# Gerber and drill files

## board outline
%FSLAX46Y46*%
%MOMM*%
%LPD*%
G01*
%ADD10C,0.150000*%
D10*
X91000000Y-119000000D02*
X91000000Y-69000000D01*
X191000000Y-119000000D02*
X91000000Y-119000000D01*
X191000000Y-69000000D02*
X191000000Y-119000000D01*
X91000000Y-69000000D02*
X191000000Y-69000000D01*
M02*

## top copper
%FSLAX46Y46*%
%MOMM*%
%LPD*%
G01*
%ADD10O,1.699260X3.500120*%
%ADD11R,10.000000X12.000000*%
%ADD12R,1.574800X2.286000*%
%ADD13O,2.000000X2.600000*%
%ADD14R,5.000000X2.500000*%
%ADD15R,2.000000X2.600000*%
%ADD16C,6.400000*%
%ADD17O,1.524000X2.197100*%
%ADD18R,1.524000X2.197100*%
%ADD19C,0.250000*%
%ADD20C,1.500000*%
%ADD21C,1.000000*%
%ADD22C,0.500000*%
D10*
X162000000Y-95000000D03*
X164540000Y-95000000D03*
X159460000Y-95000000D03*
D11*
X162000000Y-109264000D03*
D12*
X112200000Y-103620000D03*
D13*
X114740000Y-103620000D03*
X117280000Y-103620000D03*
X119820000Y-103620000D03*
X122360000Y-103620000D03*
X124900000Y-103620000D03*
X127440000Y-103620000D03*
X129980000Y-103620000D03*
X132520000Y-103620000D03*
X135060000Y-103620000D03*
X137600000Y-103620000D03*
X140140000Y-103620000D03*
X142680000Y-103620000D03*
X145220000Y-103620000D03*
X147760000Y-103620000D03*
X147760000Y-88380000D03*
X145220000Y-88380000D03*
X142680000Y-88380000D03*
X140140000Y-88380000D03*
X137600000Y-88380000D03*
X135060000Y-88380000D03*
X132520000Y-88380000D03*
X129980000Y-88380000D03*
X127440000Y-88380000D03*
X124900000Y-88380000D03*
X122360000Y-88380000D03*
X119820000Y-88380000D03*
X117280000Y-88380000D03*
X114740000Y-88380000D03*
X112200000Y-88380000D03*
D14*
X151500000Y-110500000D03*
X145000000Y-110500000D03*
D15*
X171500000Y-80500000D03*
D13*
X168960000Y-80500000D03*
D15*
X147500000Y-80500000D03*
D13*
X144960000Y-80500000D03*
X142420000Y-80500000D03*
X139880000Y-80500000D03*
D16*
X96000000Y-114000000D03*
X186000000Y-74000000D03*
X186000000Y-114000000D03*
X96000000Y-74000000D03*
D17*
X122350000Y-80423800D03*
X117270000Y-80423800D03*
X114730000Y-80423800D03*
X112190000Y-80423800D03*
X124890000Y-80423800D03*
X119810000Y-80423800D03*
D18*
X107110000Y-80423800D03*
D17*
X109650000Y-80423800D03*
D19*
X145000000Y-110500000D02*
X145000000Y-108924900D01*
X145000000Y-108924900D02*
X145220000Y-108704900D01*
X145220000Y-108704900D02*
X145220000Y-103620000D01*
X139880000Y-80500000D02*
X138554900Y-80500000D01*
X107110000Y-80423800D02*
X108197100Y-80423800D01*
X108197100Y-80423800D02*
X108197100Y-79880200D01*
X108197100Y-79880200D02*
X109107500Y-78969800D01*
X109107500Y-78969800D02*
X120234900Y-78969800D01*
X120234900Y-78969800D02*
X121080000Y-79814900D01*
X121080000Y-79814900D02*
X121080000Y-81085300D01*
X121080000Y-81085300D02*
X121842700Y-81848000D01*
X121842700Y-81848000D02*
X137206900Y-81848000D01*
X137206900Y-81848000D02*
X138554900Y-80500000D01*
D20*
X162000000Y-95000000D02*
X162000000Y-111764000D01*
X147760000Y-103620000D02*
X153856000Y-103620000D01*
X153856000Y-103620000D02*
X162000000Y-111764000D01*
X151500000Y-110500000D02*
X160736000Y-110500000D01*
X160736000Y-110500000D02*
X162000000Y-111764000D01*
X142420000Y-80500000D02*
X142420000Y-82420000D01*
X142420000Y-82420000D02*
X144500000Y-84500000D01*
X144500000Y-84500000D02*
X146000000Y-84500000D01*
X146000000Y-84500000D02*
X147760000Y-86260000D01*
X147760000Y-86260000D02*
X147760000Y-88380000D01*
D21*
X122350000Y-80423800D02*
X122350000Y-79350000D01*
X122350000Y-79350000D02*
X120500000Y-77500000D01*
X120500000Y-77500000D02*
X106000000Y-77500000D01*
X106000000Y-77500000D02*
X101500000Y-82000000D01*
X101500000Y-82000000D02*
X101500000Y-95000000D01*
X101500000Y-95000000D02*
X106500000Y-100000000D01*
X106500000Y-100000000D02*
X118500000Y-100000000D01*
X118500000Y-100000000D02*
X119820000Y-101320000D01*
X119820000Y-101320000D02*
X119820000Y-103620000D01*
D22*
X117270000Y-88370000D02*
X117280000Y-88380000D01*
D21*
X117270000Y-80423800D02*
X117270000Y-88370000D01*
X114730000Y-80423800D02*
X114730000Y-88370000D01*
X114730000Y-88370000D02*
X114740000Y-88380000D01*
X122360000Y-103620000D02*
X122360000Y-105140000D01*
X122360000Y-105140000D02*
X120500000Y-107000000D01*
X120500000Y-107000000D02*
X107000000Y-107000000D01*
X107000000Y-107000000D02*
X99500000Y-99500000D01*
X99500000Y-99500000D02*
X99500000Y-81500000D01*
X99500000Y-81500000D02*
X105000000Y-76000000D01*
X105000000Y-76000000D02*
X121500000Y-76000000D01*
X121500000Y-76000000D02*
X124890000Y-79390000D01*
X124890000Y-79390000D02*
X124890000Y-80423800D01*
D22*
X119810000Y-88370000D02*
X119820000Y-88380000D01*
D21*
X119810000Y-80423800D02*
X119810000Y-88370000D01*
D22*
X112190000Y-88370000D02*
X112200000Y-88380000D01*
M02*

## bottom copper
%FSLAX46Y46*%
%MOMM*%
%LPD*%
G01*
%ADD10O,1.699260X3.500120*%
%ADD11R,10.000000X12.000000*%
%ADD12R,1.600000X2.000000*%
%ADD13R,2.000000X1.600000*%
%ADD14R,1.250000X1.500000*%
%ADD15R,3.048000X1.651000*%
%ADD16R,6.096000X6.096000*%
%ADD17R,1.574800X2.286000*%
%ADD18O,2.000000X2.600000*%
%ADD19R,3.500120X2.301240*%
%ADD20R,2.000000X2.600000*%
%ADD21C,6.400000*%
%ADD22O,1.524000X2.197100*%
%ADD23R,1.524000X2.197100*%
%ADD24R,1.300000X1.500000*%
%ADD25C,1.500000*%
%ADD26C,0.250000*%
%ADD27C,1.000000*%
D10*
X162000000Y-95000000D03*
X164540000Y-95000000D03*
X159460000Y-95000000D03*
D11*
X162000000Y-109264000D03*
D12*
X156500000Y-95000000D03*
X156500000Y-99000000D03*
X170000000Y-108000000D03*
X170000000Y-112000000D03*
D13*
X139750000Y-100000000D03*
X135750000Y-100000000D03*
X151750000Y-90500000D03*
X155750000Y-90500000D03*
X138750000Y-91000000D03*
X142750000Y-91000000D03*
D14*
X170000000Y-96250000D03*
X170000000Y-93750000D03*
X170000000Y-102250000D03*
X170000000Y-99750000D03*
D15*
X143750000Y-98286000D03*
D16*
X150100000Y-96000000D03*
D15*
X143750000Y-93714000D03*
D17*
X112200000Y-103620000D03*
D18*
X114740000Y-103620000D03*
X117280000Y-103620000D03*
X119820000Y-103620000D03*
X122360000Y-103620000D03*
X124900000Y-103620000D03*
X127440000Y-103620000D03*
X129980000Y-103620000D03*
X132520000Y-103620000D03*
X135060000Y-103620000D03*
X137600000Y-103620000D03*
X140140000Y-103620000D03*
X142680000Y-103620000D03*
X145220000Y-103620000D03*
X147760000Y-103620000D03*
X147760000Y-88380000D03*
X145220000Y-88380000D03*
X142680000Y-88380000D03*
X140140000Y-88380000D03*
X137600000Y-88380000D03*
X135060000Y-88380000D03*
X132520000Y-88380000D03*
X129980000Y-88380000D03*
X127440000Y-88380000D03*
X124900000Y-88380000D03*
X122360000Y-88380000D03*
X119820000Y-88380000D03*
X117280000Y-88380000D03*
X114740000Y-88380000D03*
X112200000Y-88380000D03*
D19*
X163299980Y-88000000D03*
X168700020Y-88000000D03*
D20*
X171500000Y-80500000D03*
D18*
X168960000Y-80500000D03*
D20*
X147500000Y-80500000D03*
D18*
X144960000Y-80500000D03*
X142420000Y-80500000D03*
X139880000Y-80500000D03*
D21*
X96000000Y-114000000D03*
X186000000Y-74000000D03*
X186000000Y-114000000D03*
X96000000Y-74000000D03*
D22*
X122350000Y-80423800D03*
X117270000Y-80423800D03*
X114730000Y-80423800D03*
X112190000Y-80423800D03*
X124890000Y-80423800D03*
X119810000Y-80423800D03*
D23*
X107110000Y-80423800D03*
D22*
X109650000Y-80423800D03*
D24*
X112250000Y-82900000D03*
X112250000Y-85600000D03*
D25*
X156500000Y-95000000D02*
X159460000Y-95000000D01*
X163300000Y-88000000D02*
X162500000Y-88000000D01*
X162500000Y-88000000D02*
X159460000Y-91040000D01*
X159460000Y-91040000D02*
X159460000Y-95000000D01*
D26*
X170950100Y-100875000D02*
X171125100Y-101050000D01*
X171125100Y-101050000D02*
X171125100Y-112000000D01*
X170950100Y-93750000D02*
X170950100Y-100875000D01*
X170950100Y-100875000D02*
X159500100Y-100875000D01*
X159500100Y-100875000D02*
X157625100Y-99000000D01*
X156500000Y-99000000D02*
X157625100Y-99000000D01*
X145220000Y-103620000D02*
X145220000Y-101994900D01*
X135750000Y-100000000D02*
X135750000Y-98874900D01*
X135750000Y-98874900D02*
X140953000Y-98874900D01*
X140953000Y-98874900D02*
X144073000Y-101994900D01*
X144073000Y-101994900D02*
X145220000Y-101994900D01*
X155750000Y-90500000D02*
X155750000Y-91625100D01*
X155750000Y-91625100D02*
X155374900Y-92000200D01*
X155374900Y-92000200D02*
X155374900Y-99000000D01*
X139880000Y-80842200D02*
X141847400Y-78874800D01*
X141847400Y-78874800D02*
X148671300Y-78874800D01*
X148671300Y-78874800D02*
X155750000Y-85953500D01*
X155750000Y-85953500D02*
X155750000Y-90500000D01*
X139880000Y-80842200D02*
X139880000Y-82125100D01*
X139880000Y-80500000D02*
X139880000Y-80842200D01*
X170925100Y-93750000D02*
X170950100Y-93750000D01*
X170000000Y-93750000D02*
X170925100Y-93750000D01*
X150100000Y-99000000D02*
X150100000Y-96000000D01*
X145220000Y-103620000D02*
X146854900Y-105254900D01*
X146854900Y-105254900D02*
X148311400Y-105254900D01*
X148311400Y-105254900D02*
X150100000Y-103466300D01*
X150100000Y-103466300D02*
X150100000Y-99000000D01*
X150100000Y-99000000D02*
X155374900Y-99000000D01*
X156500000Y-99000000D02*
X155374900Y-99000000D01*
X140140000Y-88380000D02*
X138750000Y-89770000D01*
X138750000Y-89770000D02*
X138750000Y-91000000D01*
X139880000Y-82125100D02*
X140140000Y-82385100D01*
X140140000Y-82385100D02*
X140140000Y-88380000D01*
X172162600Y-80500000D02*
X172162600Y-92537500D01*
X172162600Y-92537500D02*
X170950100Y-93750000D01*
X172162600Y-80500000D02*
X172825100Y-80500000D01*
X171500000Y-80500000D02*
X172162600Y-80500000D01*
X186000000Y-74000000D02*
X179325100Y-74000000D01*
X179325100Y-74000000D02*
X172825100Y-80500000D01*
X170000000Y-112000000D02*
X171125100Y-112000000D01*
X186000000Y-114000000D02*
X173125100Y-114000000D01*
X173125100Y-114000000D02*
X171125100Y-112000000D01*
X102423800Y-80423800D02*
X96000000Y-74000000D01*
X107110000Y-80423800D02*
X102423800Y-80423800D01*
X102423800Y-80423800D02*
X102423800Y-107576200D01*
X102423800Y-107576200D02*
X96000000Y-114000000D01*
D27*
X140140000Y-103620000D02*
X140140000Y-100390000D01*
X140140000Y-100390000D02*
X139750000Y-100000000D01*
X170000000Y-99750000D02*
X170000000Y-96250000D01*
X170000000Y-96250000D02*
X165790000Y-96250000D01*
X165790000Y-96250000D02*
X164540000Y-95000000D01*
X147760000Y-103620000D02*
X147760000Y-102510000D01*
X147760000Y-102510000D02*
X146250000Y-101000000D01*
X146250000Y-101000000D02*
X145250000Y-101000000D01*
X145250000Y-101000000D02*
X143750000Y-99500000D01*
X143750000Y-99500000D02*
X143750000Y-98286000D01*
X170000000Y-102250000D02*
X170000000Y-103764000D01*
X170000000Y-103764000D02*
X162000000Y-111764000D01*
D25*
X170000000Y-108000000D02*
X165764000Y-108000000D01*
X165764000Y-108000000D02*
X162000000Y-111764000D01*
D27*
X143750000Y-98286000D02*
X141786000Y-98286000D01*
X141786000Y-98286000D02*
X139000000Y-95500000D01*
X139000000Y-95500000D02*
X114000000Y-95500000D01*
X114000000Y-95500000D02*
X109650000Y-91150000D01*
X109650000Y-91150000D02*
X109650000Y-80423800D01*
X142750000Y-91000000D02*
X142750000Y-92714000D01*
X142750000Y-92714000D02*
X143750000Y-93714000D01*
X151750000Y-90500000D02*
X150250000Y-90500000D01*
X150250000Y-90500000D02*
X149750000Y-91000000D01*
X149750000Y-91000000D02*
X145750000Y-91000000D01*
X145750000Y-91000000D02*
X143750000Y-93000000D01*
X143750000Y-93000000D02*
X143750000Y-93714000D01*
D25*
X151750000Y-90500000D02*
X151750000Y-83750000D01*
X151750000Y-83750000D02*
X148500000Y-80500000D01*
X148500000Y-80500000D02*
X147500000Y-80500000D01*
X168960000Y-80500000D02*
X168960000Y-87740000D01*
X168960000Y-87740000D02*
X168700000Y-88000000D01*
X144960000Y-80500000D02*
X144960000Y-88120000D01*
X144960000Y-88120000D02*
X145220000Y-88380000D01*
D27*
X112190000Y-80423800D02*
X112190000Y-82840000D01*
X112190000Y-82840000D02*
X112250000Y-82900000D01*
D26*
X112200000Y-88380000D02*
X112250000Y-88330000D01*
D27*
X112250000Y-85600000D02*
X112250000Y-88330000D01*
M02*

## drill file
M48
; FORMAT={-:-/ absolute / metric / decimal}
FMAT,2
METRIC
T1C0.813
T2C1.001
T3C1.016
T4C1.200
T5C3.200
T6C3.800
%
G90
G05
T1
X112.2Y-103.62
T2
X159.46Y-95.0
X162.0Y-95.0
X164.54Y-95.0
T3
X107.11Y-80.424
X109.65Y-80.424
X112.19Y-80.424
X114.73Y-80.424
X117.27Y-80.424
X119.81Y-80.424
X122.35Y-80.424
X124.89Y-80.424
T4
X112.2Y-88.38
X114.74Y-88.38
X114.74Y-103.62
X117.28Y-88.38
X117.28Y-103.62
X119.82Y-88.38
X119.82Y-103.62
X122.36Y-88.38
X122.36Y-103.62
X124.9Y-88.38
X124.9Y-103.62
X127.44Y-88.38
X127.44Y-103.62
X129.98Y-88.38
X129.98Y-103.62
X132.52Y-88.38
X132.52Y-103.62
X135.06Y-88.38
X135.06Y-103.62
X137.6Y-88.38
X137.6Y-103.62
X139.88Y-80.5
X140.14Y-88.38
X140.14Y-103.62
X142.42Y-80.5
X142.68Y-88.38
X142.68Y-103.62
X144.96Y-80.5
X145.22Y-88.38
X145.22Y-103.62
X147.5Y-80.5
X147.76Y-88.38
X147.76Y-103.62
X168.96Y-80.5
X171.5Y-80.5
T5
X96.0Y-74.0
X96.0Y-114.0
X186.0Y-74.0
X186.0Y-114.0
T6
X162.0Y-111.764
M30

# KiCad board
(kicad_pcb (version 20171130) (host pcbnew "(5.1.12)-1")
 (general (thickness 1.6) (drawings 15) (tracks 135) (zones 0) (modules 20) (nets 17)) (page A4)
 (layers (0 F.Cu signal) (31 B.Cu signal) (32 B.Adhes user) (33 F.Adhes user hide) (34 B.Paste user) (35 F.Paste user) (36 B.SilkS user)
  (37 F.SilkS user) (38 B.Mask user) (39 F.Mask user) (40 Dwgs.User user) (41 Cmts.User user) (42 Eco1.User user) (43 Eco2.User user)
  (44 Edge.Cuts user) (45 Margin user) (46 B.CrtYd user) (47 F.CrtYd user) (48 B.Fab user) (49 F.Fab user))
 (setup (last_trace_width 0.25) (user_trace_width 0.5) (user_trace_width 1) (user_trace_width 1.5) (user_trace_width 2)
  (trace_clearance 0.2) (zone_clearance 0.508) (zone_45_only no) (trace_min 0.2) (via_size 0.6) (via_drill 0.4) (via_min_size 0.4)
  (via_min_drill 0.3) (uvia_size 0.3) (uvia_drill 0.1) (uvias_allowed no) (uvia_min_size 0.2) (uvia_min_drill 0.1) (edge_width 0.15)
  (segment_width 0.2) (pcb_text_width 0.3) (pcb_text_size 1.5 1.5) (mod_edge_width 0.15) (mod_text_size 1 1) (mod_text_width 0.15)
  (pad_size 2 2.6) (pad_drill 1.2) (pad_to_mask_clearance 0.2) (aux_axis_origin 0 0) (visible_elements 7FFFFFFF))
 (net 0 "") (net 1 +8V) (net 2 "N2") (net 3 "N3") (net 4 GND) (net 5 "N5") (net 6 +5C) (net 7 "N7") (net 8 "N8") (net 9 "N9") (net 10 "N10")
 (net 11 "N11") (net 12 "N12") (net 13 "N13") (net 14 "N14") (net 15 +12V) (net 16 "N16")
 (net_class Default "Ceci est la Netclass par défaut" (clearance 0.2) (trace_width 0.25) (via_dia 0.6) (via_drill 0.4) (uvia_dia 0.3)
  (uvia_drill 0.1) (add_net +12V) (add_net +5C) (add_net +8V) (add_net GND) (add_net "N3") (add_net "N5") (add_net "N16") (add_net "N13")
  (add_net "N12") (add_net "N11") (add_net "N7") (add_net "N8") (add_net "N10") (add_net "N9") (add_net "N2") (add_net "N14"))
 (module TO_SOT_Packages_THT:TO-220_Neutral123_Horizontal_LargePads (layer F.Cu) (at 162 95 180)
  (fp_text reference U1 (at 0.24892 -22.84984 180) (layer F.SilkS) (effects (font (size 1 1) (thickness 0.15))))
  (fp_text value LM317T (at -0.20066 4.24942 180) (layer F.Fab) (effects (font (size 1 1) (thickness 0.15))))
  (pad 2 thru_hole oval (at 0 0 270) (size 3.50012 1.69926) (drill 1.00076) (layers *.Cu *.Mask F.SilkS) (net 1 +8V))
  (pad 1 thru_hole oval (at -2.54 0 270) (size 3.50012 1.69926) (drill 1.00076) (layers *.Cu *.Mask F.SilkS) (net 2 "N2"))
  (pad 3 thru_hole oval (at 2.54 0 270) (size 3.50012 1.69926) (drill 1.00076) (layers *.Cu *.Mask F.SilkS) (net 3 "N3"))
  (pad 2 thru_hole rect (at 0 -16.764 270) (size 12 10) (drill 3.79984 (offset -2.5 0)) (layers *.Cu *.Paste *.Mask) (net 1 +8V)))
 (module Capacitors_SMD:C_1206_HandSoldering (layer B.Cu) (at 156.5 97 270)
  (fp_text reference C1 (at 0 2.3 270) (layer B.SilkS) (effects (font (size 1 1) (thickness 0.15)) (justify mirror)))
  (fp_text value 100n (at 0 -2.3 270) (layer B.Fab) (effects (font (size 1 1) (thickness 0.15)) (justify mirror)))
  (pad 1 smd rect (at -2 0 270) (size 2 1.6) (layers B.Cu B.Paste B.Mask) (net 3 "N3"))
  (pad 2 smd rect (at 2 0 270) (size 2 1.6) (layers B.Cu B.Paste B.Mask) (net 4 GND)))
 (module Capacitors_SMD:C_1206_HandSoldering (layer B.Cu) (at 170 110 270)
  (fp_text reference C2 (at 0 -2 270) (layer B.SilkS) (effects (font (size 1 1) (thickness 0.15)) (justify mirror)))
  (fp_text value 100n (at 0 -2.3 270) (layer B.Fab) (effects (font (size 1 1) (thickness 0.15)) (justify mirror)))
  (pad 1 smd rect (at -2 0 270) (size 2 1.6) (layers B.Cu B.Paste B.Mask) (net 1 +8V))
  (pad 2 smd rect (at 2 0 270) (size 2 1.6) (layers B.Cu B.Paste B.Mask) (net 4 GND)))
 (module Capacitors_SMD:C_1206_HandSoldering (layer B.Cu) (at 137.75 100 180)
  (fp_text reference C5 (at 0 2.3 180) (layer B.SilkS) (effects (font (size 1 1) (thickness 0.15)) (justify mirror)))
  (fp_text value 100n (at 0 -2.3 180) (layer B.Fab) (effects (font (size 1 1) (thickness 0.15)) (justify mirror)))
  (pad 1 smd rect (at -2 0 180) (size 2 1.6) (layers B.Cu B.Paste B.Mask) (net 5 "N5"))
  (pad 2 smd rect (at 2 0 180) (size 2 1.6) (layers B.Cu B.Paste B.Mask) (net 4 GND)))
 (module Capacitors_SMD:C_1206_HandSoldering (layer B.Cu) (at 153.75 90.5)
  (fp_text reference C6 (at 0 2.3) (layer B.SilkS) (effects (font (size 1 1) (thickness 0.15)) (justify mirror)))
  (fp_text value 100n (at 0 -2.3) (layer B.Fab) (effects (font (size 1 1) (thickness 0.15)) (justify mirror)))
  (pad 1 smd rect (at -2 0) (size 2 1.6) (layers B.Cu B.Paste B.Mask) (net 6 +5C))
  (pad 2 smd rect (at 2 0) (size 2 1.6) (layers B.Cu B.Paste B.Mask) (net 4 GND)))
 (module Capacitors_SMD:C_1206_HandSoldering (layer B.Cu) (at 140.75 91)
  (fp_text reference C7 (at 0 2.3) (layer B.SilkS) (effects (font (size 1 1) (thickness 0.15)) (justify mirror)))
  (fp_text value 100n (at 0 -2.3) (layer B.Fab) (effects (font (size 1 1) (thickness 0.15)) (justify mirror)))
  (pad 1 smd rect (at -2 0) (size 2 1.6) (layers B.Cu B.Paste B.Mask) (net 4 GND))
  (pad 2 smd rect (at 2 0) (size 2 1.6) (layers B.Cu B.Paste B.Mask) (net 6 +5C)))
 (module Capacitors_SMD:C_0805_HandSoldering (layer B.Cu) (at 170 95 90)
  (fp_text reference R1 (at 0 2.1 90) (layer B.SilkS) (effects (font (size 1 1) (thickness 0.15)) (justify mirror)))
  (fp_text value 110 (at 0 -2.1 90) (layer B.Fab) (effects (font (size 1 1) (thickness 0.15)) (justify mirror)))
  (pad 1 smd rect (at -1.25 0 90) (size 1.5 1.25) (layers B.Cu B.Paste B.Mask) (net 2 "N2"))
  (pad 2 smd rect (at 1.25 0 90) (size 1.5 1.25) (layers B.Cu B.Paste B.Mask) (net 4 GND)))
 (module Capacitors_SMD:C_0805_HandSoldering (layer B.Cu) (at 170 101 90)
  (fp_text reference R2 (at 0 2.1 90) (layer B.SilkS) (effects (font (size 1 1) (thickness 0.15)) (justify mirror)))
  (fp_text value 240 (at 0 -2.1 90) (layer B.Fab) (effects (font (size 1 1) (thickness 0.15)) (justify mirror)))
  (pad 1 smd rect (at -1.25 0 90) (size 1.5 1.25) (layers B.Cu B.Paste B.Mask) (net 1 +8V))
  (pad 2 smd rect (at 1.25 0 90) (size 1.5 1.25) (layers B.Cu B.Paste B.Mask) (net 2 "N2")))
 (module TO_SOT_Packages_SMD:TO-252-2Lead (layer B.Cu) (at 143.75 96 90)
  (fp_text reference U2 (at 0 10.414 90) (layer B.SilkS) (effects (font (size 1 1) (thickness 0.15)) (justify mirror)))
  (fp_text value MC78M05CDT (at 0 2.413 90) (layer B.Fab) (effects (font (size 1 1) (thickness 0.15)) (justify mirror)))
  (pad 1 smd rect (at -2.286 0 90) (size 1.651 3.048) (layers B.Cu B.Paste B.Mask) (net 1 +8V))
  (pad 2 smd rect (at 0 6.35 90) (size 6.096 6.096) (layers B.Cu B.Paste B.Mask) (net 4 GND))
  (pad 3 smd rect (at 2.286 0 90) (size 1.651 3.048) (layers B.Cu B.Paste B.Mask) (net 6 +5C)))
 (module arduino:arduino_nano (layer F.Cu) (at 131.25 96)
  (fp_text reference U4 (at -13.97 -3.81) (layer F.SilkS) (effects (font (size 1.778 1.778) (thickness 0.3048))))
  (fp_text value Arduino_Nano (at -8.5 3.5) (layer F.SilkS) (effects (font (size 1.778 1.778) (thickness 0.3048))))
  (pad 1 thru_hole rect (at -19.05 7.62) (size 1.5748 2.286) (drill 0.8128) (layers *.Cu *.Mask F.SilkS))
  (pad 2 thru_hole oval (at -16.51 7.62) (size 2 2.6) (drill 1.2) (layers *.Cu *.Mask F.SilkS))
  (pad 3 thru_hole oval (at -13.97 7.62) (size 2 2.6) (drill 1.2) (layers *.Cu *.Mask F.SilkS))
  (pad 4 thru_hole oval (at -11.43 7.62) (size 2 2.6) (drill 1.2) (layers *.Cu *.Mask F.SilkS) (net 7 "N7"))
  (pad 5 thru_hole oval (at -8.89 7.62) (size 2 2.6) (drill 1.2) (layers *.Cu *.Mask F.SilkS) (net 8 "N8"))
  (pad 6 thru_hole oval (at -6.35 7.62) (size 2 2.6) (drill 1.2) (layers *.Cu *.Mask F.SilkS))
  (pad 7 thru_hole oval (at -3.81 7.62) (size 2 2.6) (drill 1.2) (layers *.Cu *.Mask F.SilkS))
  (pad 8 thru_hole oval (at -1.27 7.62) (size 2 2.6) (drill 1.2) (layers *.Cu *.Mask F.SilkS))
  (pad 9 thru_hole oval (at 1.27 7.62) (size 2 2.6) (drill 1.2) (layers *.Cu *.Mask F.SilkS))
  (pad 10 thru_hole oval (at 3.81 7.62) (size 2 2.6) (drill 1.2) (layers *.Cu *.Mask F.SilkS))
  (pad 11 thru_hole oval (at 6.35 7.62) (size 2 2.6) (drill 1.2) (layers *.Cu *.Mask F.SilkS))
  (pad 12 thru_hole oval (at 8.89 7.62) (size 2 2.6) (drill 1.2) (layers *.Cu *.Mask F.SilkS) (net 5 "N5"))
  (pad 13 thru_hole oval (at 11.43 7.62) (size 2 2.6) (drill 1.2) (layers *.Cu *.Mask F.SilkS))
  (pad 14 thru_hole oval (at 13.97 7.62) (size 2 2.6) (drill 1.2) (layers *.Cu *.Mask F.SilkS) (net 4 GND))
  (pad 15 thru_hole oval (at 16.51 7.62) (size 2 2.6) (drill 1.2) (layers *.Cu *.Mask F.SilkS) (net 1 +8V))
  (pad 16 thru_hole oval (at 16.51 -7.62) (size 2 2.6) (drill 1.2) (layers *.Cu *.Mask F.SilkS) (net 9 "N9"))
  (pad 17 thru_hole oval (at 13.97 -7.62) (size 2 2.6) (drill 1.2) (layers *.Cu *.Mask F.SilkS) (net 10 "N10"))
  (pad 18 thru_hole oval (at 11.43 -7.62) (size 2 2.6) (drill 1.2) (layers *.Cu *.Mask F.SilkS))
  (pad 19 thru_hole oval (at 8.89 -7.62) (size 2 2.6) (drill 1.2) (layers *.Cu *.Mask F.SilkS) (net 4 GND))
  (pad 20 thru_hole oval (at 6.35 -7.62) (size 2 2.6) (drill 1.2) (layers *.Cu *.Mask F.SilkS))
  (pad 21 thru_hole oval (at 3.81 -7.62) (size 2 2.6) (drill 1.2) (layers *.Cu *.Mask F.SilkS))
  (pad 22 thru_hole oval (at 1.27 -7.62) (size 2 2.6) (drill 1.2) (layers *.Cu *.Mask F.SilkS))
  (pad 23 thru_hole oval (at -1.27 -7.62) (size 2 2.6) (drill 1.2) (layers *.Cu *.Mask F.SilkS))
  (pad 24 thru_hole oval (at -3.81 -7.62) (size 2 2.6) (drill 1.2) (layers *.Cu *.Mask F.SilkS))
  (pad 25 thru_hole oval (at -6.35 -7.62) (size 2 2.6) (drill 1.2) (layers *.Cu *.Mask F.SilkS))
  (pad 26 thru_hole oval (at -8.89 -7.62) (size 2 2.6) (drill 1.2) (layers *.Cu *.Mask F.SilkS))
  (pad 27 thru_hole oval (at -11.43 -7.62) (size 2 2.6) (drill 1.2) (layers *.Cu *.Mask F.SilkS) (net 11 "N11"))
  (pad 28 thru_hole oval (at -13.97 -7.62) (size 2 2.6) (drill 1.2) (layers *.Cu *.Mask F.SilkS) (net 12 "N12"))
  (pad 29 thru_hole oval (at -16.51 -7.62) (size 2 2.6) (drill 1.2) (layers *.Cu *.Mask F.SilkS) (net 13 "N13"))
  (pad 30 thru_hole oval (at -19.05 -7.62) (size 2 2.6) (drill 1.2) (layers *.Cu *.Mask F.SilkS) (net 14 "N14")))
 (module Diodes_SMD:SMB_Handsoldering (layer B.Cu) (at 166 88)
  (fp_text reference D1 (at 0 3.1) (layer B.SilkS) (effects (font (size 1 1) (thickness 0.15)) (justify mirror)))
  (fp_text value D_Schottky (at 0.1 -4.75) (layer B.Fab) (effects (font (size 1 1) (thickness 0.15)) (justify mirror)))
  (pad 1 smd rect (at -2.70002 0) (size 3.50012 2.30124) (layers B.Cu B.Paste B.Mask) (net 3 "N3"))
  (pad 2 smd rect (at 2.70002 0) (size 3.50012 2.30124) (layers B.Cu B.Paste B.Mask) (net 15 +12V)))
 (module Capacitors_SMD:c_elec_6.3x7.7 (layer F.Cu) (at 148.5 110.5)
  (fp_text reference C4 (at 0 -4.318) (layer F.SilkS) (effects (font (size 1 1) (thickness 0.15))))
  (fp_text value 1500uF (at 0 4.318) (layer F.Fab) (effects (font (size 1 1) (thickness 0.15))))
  (pad 1 smd rect (at 3 0) (size 5 2.5) (layers F.Cu F.Paste F.Mask) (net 1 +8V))
  (pad 2 smd rect (at -3.5 0) (size 5 2.5) (layers F.Cu F.Paste F.Mask) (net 4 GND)))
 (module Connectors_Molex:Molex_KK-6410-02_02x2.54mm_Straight (layer F.Cu) (at 171.5 80.5 180)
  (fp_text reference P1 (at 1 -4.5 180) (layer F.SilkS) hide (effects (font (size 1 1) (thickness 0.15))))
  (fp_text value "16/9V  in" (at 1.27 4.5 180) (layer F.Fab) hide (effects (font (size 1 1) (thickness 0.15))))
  (pad 1 thru_hole rect (at 0 0 180) (size 2 2.6) (drill 1.2) (layers *.Cu *.Mask) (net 4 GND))
  (pad 2 thru_hole oval (at 2.54 0 180) (size 2 2.6) (drill 1.2) (layers *.Cu *.Mask) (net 15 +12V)))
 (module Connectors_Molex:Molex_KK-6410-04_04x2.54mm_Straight (layer F.Cu) (at 147.5 80.5 180)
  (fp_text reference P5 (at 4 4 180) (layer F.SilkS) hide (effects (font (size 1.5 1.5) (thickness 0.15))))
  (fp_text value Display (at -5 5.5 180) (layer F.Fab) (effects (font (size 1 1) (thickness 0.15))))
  (pad 1 thru_hole rect (at 0 0 180) (size 2 2.6) (drill 1.2) (layers *.Cu *.Mask) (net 6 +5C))
  (pad 2 thru_hole oval (at 2.54 0 180) (size 2 2.6) (drill 1.2) (layers *.Cu *.Mask) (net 10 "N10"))
  (pad 3 thru_hole oval (at 5.08 0 180) (size 2 2.6) (drill 1.2) (layers *.Cu *.Mask) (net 9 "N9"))
  (pad 4 thru_hole oval (at 7.62 0 180) (size 2 2.6) (drill 1.2) (layers *.Cu *.Mask) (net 4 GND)))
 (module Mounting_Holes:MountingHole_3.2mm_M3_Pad (layer F.Cu) (at 96 114)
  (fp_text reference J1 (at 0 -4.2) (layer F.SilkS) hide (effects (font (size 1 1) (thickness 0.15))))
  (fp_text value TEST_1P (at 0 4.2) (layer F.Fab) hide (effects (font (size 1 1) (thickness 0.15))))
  (pad 1 thru_hole circle (at 0 0) (size 6.4 6.4) (drill 3.2) (layers *.Cu *.Mask) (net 4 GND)))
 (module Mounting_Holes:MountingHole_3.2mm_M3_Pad (layer F.Cu) (at 186 74)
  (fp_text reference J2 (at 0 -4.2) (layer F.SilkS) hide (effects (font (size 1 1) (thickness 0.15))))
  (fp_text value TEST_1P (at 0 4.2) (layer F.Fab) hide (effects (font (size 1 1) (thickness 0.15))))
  (pad 1 thru_hole circle (at 0 0) (size 6.4 6.4) (drill 3.2) (layers *.Cu *.Mask) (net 4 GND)))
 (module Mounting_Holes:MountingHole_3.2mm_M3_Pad (layer F.Cu) (at 186 114)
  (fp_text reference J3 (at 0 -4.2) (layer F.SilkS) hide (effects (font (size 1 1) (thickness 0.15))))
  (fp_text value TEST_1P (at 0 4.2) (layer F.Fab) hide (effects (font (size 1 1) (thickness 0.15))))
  (pad 1 thru_hole circle (at 0 0) (size 6.4 6.4) (drill 3.2) (layers *.Cu *.Mask) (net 4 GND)))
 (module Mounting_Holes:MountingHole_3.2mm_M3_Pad (layer F.Cu) (at 96 74)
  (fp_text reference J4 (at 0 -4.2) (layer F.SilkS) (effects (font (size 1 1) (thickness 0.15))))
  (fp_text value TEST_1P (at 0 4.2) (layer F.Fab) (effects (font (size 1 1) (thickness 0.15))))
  (pad 1 thru_hole circle (at 0 0) (size 6.4 6.4) (drill 3.2) (layers *.Cu *.Mask) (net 4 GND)))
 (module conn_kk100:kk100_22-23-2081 (layer F.Cu) (at 116 80.5)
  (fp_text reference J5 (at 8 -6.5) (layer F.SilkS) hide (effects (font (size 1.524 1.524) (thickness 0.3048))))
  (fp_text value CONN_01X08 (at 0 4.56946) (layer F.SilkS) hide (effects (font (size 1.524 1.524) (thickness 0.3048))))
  (pad 7 thru_hole oval (at 6.35 -0.0762) (size 1.524 2.1971) (drill 1.016) (layers *.Cu *.Mask F.SilkS) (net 7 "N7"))
  (pad 5 thru_hole oval (at 1.27 -0.0762) (size 1.524 2.1971) (drill 1.016) (layers *.Cu *.Mask F.SilkS) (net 12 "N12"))
  (pad 4 thru_hole oval (at -1.27 -0.0762) (size 1.524 2.1971) (drill 1.016) (layers *.Cu *.Mask F.SilkS) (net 13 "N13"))
  (pad 3 thru_hole oval (at -3.81 -0.0762) (size 1.524 2.1971) (drill 1.016) (layers *.Cu *.Mask F.SilkS) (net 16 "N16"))
  (pad 8 thru_hole oval (at 8.89 -0.0762) (size 1.524 2.1971) (drill 1.016) (layers *.Cu *.Mask F.SilkS) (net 8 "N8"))
  (pad 6 thru_hole oval (at 3.81 -0.0762) (size 1.524 2.1971) (drill 1.016) (layers *.Cu *.Mask F.SilkS) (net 11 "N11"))
  (pad 1 thru_hole rect (at -8.89 -0.0762) (size 1.524 2.1971) (drill 1.016) (layers *.Cu *.Mask F.SilkS) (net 4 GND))
  (pad 2 thru_hole oval (at -6.35 -0.0762) (size 1.524 2.1971) (drill 1.016) (layers *.Cu *.Mask F.SilkS) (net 1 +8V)))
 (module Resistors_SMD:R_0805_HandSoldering (layer B.Cu) (at 112.25 84.25 270)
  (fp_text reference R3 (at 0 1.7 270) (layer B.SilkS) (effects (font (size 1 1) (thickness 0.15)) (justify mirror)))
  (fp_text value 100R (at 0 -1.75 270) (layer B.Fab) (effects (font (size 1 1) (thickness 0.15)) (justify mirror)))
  (pad 1 smd rect (at -1.35 0 270) (size 1.5 1.3) (layers B.Cu B.Paste B.Mask) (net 16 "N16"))
  (pad 2 smd rect (at 1.35 0 270) (size 1.5 1.3) (layers B.Cu B.Paste B.Mask) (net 14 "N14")))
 (gr_line (start 91 119) (end 91 69) (angle 90) (layer Edge.Cuts) (width 0.15))
 (gr_line (start 191 119) (end 91 119) (angle 90) (layer Edge.Cuts) (width 0.15))
 (gr_line (start 191 69) (end 191 119) (angle 90) (layer Edge.Cuts) (width 0.15))
 (gr_line (start 91 69) (end 191 69) (angle 90) (layer Edge.Cuts) (width 0.15))
 (segment (start 156.5 95) (end 159.46 95) (width 1.5) (layer B.Cu) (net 3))
 (segment (start 163.3 88) (end 162.5 88) (width 1.5) (layer B.Cu) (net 3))
 (segment (start 162.5 88) (end 159.46 91.04) (width 1.5) (layer B.Cu) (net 3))
 (segment (start 159.46 91.04) (end 159.46 95) (width 1.5) (layer B.Cu) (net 3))
 (segment (start 170.9501 100.875) (end 171.1251 101.05) (width 0.25) (layer B.Cu) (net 4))
 (segment (start 171.1251 101.05) (end 171.1251 112) (width 0.25) (layer B.Cu) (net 4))
 (segment (start 170.9501 93.75) (end 170.9501 100.875) (width 0.25) (layer B.Cu) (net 4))
 (segment (start 170.9501 100.875) (end 159.5001 100.875) (width 0.25) (layer B.Cu) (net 4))
 (segment (start 159.5001 100.875) (end 157.6251 99) (width 0.25) (layer B.Cu) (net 4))
 (segment (start 156.5 99) (end 157.6251 99) (width 0.25) (layer B.Cu) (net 4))
 (segment (start 145.22 103.62) (end 145.22 101.9949) (width 0.25) (layer B.Cu) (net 4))
 (segment (start 135.75 100) (end 135.75 98.8749) (width 0.25) (layer B.Cu) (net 4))
 (segment (start 135.75 98.8749) (end 140.953 98.8749) (width 0.25) (layer B.Cu) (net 4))
 (segment (start 140.953 98.8749) (end 144.073 101.9949) (width 0.25) (layer B.Cu) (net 4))
 (segment (start 144.073 101.9949) (end 145.22 101.9949) (width 0.25) (layer B.Cu) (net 4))
 (segment (start 155.75 90.5) (end 155.75 91.6251) (width 0.25) (layer B.Cu) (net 4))
 (segment (start 155.75 91.6251) (end 155.3749 92.0002) (width 0.25) (layer B.Cu) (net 4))
 (segment (start 155.3749 92.0002) (end 155.3749 99) (width 0.25) (layer B.Cu) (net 4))
 (segment (start 139.88 80.8422) (end 141.8474 78.8748) (width 0.25) (layer B.Cu) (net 4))
 (segment (start 141.8474 78.8748) (end 148.6713 78.8748) (width 0.25) (layer B.Cu) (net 4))
 (segment (start 148.6713 78.8748) (end 155.75 85.9535) (width 0.25) (layer B.Cu) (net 4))
 (segment (start 155.75 85.9535) (end 155.75 90.5) (width 0.25) (layer B.Cu) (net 4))
 (segment (start 139.88 80.8422) (end 139.88 82.1251) (width 0.25) (layer B.Cu) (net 4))
 (segment (start 139.88 80.5) (end 139.88 80.8422) (width 0.25) (layer B.Cu) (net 4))
 (segment (start 170.9251 93.75) (end 170.9501 93.75) (width 0.25) (layer B.Cu) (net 4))
 (segment (start 170 93.75) (end 170.9251 93.75) (width 0.25) (layer B.Cu) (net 4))
 (segment (start 150.1 99) (end 150.1 96) (width 0.25) (layer B.Cu) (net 4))
 (segment (start 145.22 103.62) (end 146.8549 105.2549) (width 0.25) (layer B.Cu) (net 4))
 (segment (start 146.8549 105.2549) (end 148.3114 105.2549) (width 0.25) (layer B.Cu) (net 4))
 (segment (start 148.3114 105.2549) (end 150.1 103.4663) (width 0.25) (layer B.Cu) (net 4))
 (segment (start 150.1 103.4663) (end 150.1 99) (width 0.25) (layer B.Cu) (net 4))
 (segment (start 150.1 99) (end 155.3749 99) (width 0.25) (layer B.Cu) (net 4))
 (segment (start 156.5 99) (end 155.3749 99) (width 0.25) (layer B.Cu) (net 4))
 (segment (start 140.14 88.38) (end 138.75 89.77) (width 0.25) (layer B.Cu) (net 4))
 (segment (start 138.75 89.77) (end 138.75 91) (width 0.25) (layer B.Cu) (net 4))
 (segment (start 139.88 82.1251) (end 140.14 82.3851) (width 0.25) (layer B.Cu) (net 4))
 (segment (start 140.14 82.3851) (end 140.14 88.38) (width 0.25) (layer B.Cu) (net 4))
 (segment (start 145 110.5) (end 145 108.9249) (width 0.25) (layer F.Cu) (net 4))
 (segment (start 145 108.9249) (end 145.22 108.7049) (width 0.25) (layer F.Cu) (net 4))
 (segment (start 145.22 108.7049) (end 145.22 103.62) (width 0.25) (layer F.Cu) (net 4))
 (segment (start 172.1626 80.5) (end 172.1626 92.5375) (width 0.25) (layer B.Cu) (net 4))
 (segment (start 172.1626 92.5375) (end 170.9501 93.75) (width 0.25) (layer B.Cu) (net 4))
 (segment (start 172.1626 80.5) (end 172.8251 80.5) (width 0.25) (layer B.Cu) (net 4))
 (segment (start 171.5 80.5) (end 172.1626 80.5) (width 0.25) (layer B.Cu) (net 4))
 (segment (start 139.88 80.5) (end 138.5549 80.5) (width 0.25) (layer F.Cu) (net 4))
 (segment (start 107.11 80.4238) (end 108.1971 80.4238) (width 0.25) (layer F.Cu) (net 4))
 (segment (start 108.1971 80.4238) (end 108.1971 79.8802) (width 0.25) (layer F.Cu) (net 4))
 (segment (start 108.1971 79.8802) (end 109.1075 78.9698) (width 0.25) (layer F.Cu) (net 4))
 (segment (start 109.1075 78.9698) (end 120.2349 78.9698) (width 0.25) (layer F.Cu) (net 4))
 (segment (start 120.2349 78.9698) (end 121.08 79.8149) (width 0.25) (layer F.Cu) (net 4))
 (segment (start 121.08 79.8149) (end 121.08 81.0853) (width 0.25) (layer F.Cu) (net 4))
 (segment (start 121.08 81.0853) (end 121.8427 81.848) (width 0.25) (layer F.Cu) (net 4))
 (segment (start 121.8427 81.848) (end 137.2069 81.848) (width 0.25) (layer F.Cu) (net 4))
 (segment (start 137.2069 81.848) (end 138.5549 80.5) (width 0.25) (layer F.Cu) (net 4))
 (segment (start 186 74) (end 179.3251 74) (width 0.25) (layer B.Cu) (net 4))
 (segment (start 179.3251 74) (end 172.8251 80.5) (width 0.25) (layer B.Cu) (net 4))
 (segment (start 170 112) (end 171.1251 112) (width 0.25) (layer B.Cu) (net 4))
 (segment (start 186 114) (end 173.1251 114) (width 0.25) (layer B.Cu) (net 4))
 (segment (start 173.1251 114) (end 171.1251 112) (width 0.25) (layer B.Cu) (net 4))
 (segment (start 102.4238 80.4238) (end 96 74) (width 0.25) (layer B.Cu) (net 4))
 (segment (start 107.11 80.4238) (end 102.4238 80.4238) (width 0.25) (layer B.Cu) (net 4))
 (segment (start 102.4238 80.4238) (end 102.4238 107.5762) (width 0.25) (layer B.Cu) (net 4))
 (segment (start 102.4238 107.5762) (end 96 114) (width 0.25) (layer B.Cu) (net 4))
 (segment (start 140.14 103.62) (end 140.14 100.39) (width 1) (layer B.Cu) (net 5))
 (segment (start 140.14 100.39) (end 139.75 100) (width 1) (layer B.Cu) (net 5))
 (segment (start 170 99.75) (end 170 96.25) (width 1) (layer B.Cu) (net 2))
 (segment (start 170 96.25) (end 165.79 96.25) (width 1) (layer B.Cu) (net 2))
 (segment (start 165.79 96.25) (end 164.54 95) (width 1) (layer B.Cu) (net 2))
 (segment (start 147.76 103.62) (end 147.76 102.51) (width 1) (layer B.Cu) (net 1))
 (segment (start 147.76 102.51) (end 146.25 101) (width 1) (layer B.Cu) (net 1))
 (segment (start 146.25 101) (end 145.25 101) (width 1) (layer B.Cu) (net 1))
 (segment (start 145.25 101) (end 143.75 99.5) (width 1) (layer B.Cu) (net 1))
 (segment (start 143.75 99.5) (end 143.75 98.286) (width 1) (layer B.Cu) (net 1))
 (segment (start 162 95) (end 162 111.764) (width 1.5) (layer F.Cu) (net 1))
 (segment (start 170 102.25) (end 170 103.764) (width 1) (layer B.Cu) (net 1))
 (segment (start 170 103.764) (end 162 111.764) (width 1) (layer B.Cu) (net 1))
 (segment (start 147.76 103.62) (end 153.856 103.62) (width 1.5) (layer F.Cu) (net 1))
 (segment (start 153.856 103.62) (end 162 111.764) (width 1.5) (layer F.Cu) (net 1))
 (segment (start 170 108) (end 165.764 108) (width 1.5) (layer B.Cu) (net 1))
 (segment (start 165.764 108) (end 162 111.764) (width 1.5) (layer B.Cu) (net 1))
 (segment (start 143.75 98.286) (end 141.786 98.286) (width 1) (layer B.Cu) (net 1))
 (segment (start 141.786 98.286) (end 139 95.5) (width 1) (layer B.Cu) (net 1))
 (segment (start 139 95.5) (end 114 95.5) (width 1) (layer B.Cu) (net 1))
 (segment (start 114 95.5) (end 109.65 91.15) (width 1) (layer B.Cu) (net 1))
 (segment (start 109.65 91.15) (end 109.65 80.4238) (width 1) (layer B.Cu) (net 1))
 (segment (start 151.5 110.5) (end 160.736 110.5) (width 1.5) (layer F.Cu) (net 1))
 (segment (start 160.736 110.5) (end 162 111.764) (width 1.5) (layer F.Cu) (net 1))
 (segment (start 142.75 91) (end 142.75 92.714) (width 1) (layer B.Cu) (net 6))
 (segment (start 142.75 92.714) (end 143.75 93.714) (width 1) (layer B.Cu) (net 6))
 (segment (start 151.75 90.5) (end 150.25 90.5) (width 1) (layer B.Cu) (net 6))
 (segment (start 150.25 90.5) (end 149.75 91) (width 1) (layer B.Cu) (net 6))
 (segment (start 149.75 91) (end 145.75 91) (width 1) (layer B.Cu) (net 6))
 (segment (start 145.75 91) (end 143.75 93) (width 1) (layer B.Cu) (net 6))
 (segment (start 143.75 93) (end 143.75 93.714) (width 1) (layer B.Cu) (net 6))
 (segment (start 151.75 90.5) (end 151.75 83.75) (width 1.5) (layer B.Cu) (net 6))
 (segment (start 151.75 83.75) (end 148.5 80.5) (width 1.5) (layer B.Cu) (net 6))
 (segment (start 148.5 80.5) (end 147.5 80.5) (width 1.5) (layer B.Cu) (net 6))
 (segment (start 168.96 80.5) (end 168.96 87.74) (width 1.5) (layer B.Cu) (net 15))
 (segment (start 168.96 87.74) (end 168.7 88) (width 1.5) (layer B.Cu) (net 15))
 (segment (start 144.96 80.5) (end 144.96 88.12) (width 1.5) (layer B.Cu) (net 10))
 (segment (start 144.96 88.12) (end 145.22 88.38) (width 1.5) (layer B.Cu) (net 10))
 (segment (start 142.42 80.5) (end 142.42 82.42) (width 1.5) (layer F.Cu) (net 9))
 (segment (start 142.42 82.42) (end 144.5 84.5) (width 1.5) (layer F.Cu) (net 9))
 (segment (start 144.5 84.5) (end 146 84.5) (width 1.5) (layer F.Cu) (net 9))
 (segment (start 146 84.5) (end 147.76 86.26) (width 1.5) (layer F.Cu) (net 9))
 (segment (start 147.76 86.26) (end 147.76 88.38) (width 1.5) (layer F.Cu) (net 9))
 (segment (start 122.35 80.4238) (end 122.35 79.35) (width 1) (layer F.Cu) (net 7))
 (segment (start 122.35 79.35) (end 120.5 77.5) (width 1) (layer F.Cu) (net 7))
 (segment (start 120.5 77.5) (end 106 77.5) (width 1) (layer F.Cu) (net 7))
 (segment (start 106 77.5) (end 101.5 82) (width 1) (layer F.Cu) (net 7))
 (segment (start 101.5 82) (end 101.5 95) (width 1) (layer F.Cu) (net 7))
 (segment (start 101.5 95) (end 106.5 100) (width 1) (layer F.Cu) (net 7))
 (segment (start 106.5 100) (end 118.5 100) (width 1) (layer F.Cu) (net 7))
 (segment (start 118.5 100) (end 119.82 101.32) (width 1) (layer F.Cu) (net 7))
 (segment (start 119.82 101.32) (end 119.82 103.62) (width 1) (layer F.Cu) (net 7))
 (segment (start 117.27 88.37) (end 117.28 88.38) (width 0.5) (layer F.Cu) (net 12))
 (segment (start 117.27 80.4238) (end 117.27 88.37) (width 1) (layer F.Cu) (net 12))
 (segment (start 114.73 80.4238) (end 114.73 88.37) (width 1) (layer F.Cu) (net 13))
 (segment (start 114.73 88.37) (end 114.74 88.38) (width 1) (layer F.Cu) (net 13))
 (segment (start 112.19 80.4238) (end 112.19 82.84) (width 1) (layer B.Cu) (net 16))
 (segment (start 112.19 82.84) (end 112.25 82.9) (width 1) (layer B.Cu) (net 16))
 (segment (start 122.36 103.62) (end 122.36 105.14) (width 1) (layer F.Cu) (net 8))
 (segment (start 122.36 105.14) (end 120.5 107) (width 1) (layer F.Cu) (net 8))
 (segment (start 120.5 107) (end 107 107) (width 1) (layer F.Cu) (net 8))
 (segment (start 107 107) (end 99.5 99.5) (width 1) (layer F.Cu) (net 8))
 (segment (start 99.5 99.5) (end 99.5 81.5) (width 1) (layer F.Cu) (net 8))
 (segment (start 99.5 81.5) (end 105 76) (width 1) (layer F.Cu) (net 8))
 (segment (start 105 76) (end 121.5 76) (width 1) (layer F.Cu) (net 8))
 (segment (start 121.5 76) (end 124.89 79.39) (width 1) (layer F.Cu) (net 8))
 (segment (start 124.89 79.39) (end 124.89 80.4238) (width 1) (layer F.Cu) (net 8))
 (segment (start 119.81 88.37) (end 119.82 88.38) (width 0.5) (layer F.Cu) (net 11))
 (segment (start 119.81 80.4238) (end 119.81 88.37) (width 1) (layer F.Cu) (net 11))
 (segment (start 112.2 88.38) (end 112.25 88.33) (width 0.25) (layer B.Cu) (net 14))
 (segment (start 112.19 88.37) (end 112.2 88.38) (width 0.5) (layer F.Cu) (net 14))
 (segment (start 112.25 85.6) (end 112.25 88.33) (width 1) (layer B.Cu) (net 14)))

